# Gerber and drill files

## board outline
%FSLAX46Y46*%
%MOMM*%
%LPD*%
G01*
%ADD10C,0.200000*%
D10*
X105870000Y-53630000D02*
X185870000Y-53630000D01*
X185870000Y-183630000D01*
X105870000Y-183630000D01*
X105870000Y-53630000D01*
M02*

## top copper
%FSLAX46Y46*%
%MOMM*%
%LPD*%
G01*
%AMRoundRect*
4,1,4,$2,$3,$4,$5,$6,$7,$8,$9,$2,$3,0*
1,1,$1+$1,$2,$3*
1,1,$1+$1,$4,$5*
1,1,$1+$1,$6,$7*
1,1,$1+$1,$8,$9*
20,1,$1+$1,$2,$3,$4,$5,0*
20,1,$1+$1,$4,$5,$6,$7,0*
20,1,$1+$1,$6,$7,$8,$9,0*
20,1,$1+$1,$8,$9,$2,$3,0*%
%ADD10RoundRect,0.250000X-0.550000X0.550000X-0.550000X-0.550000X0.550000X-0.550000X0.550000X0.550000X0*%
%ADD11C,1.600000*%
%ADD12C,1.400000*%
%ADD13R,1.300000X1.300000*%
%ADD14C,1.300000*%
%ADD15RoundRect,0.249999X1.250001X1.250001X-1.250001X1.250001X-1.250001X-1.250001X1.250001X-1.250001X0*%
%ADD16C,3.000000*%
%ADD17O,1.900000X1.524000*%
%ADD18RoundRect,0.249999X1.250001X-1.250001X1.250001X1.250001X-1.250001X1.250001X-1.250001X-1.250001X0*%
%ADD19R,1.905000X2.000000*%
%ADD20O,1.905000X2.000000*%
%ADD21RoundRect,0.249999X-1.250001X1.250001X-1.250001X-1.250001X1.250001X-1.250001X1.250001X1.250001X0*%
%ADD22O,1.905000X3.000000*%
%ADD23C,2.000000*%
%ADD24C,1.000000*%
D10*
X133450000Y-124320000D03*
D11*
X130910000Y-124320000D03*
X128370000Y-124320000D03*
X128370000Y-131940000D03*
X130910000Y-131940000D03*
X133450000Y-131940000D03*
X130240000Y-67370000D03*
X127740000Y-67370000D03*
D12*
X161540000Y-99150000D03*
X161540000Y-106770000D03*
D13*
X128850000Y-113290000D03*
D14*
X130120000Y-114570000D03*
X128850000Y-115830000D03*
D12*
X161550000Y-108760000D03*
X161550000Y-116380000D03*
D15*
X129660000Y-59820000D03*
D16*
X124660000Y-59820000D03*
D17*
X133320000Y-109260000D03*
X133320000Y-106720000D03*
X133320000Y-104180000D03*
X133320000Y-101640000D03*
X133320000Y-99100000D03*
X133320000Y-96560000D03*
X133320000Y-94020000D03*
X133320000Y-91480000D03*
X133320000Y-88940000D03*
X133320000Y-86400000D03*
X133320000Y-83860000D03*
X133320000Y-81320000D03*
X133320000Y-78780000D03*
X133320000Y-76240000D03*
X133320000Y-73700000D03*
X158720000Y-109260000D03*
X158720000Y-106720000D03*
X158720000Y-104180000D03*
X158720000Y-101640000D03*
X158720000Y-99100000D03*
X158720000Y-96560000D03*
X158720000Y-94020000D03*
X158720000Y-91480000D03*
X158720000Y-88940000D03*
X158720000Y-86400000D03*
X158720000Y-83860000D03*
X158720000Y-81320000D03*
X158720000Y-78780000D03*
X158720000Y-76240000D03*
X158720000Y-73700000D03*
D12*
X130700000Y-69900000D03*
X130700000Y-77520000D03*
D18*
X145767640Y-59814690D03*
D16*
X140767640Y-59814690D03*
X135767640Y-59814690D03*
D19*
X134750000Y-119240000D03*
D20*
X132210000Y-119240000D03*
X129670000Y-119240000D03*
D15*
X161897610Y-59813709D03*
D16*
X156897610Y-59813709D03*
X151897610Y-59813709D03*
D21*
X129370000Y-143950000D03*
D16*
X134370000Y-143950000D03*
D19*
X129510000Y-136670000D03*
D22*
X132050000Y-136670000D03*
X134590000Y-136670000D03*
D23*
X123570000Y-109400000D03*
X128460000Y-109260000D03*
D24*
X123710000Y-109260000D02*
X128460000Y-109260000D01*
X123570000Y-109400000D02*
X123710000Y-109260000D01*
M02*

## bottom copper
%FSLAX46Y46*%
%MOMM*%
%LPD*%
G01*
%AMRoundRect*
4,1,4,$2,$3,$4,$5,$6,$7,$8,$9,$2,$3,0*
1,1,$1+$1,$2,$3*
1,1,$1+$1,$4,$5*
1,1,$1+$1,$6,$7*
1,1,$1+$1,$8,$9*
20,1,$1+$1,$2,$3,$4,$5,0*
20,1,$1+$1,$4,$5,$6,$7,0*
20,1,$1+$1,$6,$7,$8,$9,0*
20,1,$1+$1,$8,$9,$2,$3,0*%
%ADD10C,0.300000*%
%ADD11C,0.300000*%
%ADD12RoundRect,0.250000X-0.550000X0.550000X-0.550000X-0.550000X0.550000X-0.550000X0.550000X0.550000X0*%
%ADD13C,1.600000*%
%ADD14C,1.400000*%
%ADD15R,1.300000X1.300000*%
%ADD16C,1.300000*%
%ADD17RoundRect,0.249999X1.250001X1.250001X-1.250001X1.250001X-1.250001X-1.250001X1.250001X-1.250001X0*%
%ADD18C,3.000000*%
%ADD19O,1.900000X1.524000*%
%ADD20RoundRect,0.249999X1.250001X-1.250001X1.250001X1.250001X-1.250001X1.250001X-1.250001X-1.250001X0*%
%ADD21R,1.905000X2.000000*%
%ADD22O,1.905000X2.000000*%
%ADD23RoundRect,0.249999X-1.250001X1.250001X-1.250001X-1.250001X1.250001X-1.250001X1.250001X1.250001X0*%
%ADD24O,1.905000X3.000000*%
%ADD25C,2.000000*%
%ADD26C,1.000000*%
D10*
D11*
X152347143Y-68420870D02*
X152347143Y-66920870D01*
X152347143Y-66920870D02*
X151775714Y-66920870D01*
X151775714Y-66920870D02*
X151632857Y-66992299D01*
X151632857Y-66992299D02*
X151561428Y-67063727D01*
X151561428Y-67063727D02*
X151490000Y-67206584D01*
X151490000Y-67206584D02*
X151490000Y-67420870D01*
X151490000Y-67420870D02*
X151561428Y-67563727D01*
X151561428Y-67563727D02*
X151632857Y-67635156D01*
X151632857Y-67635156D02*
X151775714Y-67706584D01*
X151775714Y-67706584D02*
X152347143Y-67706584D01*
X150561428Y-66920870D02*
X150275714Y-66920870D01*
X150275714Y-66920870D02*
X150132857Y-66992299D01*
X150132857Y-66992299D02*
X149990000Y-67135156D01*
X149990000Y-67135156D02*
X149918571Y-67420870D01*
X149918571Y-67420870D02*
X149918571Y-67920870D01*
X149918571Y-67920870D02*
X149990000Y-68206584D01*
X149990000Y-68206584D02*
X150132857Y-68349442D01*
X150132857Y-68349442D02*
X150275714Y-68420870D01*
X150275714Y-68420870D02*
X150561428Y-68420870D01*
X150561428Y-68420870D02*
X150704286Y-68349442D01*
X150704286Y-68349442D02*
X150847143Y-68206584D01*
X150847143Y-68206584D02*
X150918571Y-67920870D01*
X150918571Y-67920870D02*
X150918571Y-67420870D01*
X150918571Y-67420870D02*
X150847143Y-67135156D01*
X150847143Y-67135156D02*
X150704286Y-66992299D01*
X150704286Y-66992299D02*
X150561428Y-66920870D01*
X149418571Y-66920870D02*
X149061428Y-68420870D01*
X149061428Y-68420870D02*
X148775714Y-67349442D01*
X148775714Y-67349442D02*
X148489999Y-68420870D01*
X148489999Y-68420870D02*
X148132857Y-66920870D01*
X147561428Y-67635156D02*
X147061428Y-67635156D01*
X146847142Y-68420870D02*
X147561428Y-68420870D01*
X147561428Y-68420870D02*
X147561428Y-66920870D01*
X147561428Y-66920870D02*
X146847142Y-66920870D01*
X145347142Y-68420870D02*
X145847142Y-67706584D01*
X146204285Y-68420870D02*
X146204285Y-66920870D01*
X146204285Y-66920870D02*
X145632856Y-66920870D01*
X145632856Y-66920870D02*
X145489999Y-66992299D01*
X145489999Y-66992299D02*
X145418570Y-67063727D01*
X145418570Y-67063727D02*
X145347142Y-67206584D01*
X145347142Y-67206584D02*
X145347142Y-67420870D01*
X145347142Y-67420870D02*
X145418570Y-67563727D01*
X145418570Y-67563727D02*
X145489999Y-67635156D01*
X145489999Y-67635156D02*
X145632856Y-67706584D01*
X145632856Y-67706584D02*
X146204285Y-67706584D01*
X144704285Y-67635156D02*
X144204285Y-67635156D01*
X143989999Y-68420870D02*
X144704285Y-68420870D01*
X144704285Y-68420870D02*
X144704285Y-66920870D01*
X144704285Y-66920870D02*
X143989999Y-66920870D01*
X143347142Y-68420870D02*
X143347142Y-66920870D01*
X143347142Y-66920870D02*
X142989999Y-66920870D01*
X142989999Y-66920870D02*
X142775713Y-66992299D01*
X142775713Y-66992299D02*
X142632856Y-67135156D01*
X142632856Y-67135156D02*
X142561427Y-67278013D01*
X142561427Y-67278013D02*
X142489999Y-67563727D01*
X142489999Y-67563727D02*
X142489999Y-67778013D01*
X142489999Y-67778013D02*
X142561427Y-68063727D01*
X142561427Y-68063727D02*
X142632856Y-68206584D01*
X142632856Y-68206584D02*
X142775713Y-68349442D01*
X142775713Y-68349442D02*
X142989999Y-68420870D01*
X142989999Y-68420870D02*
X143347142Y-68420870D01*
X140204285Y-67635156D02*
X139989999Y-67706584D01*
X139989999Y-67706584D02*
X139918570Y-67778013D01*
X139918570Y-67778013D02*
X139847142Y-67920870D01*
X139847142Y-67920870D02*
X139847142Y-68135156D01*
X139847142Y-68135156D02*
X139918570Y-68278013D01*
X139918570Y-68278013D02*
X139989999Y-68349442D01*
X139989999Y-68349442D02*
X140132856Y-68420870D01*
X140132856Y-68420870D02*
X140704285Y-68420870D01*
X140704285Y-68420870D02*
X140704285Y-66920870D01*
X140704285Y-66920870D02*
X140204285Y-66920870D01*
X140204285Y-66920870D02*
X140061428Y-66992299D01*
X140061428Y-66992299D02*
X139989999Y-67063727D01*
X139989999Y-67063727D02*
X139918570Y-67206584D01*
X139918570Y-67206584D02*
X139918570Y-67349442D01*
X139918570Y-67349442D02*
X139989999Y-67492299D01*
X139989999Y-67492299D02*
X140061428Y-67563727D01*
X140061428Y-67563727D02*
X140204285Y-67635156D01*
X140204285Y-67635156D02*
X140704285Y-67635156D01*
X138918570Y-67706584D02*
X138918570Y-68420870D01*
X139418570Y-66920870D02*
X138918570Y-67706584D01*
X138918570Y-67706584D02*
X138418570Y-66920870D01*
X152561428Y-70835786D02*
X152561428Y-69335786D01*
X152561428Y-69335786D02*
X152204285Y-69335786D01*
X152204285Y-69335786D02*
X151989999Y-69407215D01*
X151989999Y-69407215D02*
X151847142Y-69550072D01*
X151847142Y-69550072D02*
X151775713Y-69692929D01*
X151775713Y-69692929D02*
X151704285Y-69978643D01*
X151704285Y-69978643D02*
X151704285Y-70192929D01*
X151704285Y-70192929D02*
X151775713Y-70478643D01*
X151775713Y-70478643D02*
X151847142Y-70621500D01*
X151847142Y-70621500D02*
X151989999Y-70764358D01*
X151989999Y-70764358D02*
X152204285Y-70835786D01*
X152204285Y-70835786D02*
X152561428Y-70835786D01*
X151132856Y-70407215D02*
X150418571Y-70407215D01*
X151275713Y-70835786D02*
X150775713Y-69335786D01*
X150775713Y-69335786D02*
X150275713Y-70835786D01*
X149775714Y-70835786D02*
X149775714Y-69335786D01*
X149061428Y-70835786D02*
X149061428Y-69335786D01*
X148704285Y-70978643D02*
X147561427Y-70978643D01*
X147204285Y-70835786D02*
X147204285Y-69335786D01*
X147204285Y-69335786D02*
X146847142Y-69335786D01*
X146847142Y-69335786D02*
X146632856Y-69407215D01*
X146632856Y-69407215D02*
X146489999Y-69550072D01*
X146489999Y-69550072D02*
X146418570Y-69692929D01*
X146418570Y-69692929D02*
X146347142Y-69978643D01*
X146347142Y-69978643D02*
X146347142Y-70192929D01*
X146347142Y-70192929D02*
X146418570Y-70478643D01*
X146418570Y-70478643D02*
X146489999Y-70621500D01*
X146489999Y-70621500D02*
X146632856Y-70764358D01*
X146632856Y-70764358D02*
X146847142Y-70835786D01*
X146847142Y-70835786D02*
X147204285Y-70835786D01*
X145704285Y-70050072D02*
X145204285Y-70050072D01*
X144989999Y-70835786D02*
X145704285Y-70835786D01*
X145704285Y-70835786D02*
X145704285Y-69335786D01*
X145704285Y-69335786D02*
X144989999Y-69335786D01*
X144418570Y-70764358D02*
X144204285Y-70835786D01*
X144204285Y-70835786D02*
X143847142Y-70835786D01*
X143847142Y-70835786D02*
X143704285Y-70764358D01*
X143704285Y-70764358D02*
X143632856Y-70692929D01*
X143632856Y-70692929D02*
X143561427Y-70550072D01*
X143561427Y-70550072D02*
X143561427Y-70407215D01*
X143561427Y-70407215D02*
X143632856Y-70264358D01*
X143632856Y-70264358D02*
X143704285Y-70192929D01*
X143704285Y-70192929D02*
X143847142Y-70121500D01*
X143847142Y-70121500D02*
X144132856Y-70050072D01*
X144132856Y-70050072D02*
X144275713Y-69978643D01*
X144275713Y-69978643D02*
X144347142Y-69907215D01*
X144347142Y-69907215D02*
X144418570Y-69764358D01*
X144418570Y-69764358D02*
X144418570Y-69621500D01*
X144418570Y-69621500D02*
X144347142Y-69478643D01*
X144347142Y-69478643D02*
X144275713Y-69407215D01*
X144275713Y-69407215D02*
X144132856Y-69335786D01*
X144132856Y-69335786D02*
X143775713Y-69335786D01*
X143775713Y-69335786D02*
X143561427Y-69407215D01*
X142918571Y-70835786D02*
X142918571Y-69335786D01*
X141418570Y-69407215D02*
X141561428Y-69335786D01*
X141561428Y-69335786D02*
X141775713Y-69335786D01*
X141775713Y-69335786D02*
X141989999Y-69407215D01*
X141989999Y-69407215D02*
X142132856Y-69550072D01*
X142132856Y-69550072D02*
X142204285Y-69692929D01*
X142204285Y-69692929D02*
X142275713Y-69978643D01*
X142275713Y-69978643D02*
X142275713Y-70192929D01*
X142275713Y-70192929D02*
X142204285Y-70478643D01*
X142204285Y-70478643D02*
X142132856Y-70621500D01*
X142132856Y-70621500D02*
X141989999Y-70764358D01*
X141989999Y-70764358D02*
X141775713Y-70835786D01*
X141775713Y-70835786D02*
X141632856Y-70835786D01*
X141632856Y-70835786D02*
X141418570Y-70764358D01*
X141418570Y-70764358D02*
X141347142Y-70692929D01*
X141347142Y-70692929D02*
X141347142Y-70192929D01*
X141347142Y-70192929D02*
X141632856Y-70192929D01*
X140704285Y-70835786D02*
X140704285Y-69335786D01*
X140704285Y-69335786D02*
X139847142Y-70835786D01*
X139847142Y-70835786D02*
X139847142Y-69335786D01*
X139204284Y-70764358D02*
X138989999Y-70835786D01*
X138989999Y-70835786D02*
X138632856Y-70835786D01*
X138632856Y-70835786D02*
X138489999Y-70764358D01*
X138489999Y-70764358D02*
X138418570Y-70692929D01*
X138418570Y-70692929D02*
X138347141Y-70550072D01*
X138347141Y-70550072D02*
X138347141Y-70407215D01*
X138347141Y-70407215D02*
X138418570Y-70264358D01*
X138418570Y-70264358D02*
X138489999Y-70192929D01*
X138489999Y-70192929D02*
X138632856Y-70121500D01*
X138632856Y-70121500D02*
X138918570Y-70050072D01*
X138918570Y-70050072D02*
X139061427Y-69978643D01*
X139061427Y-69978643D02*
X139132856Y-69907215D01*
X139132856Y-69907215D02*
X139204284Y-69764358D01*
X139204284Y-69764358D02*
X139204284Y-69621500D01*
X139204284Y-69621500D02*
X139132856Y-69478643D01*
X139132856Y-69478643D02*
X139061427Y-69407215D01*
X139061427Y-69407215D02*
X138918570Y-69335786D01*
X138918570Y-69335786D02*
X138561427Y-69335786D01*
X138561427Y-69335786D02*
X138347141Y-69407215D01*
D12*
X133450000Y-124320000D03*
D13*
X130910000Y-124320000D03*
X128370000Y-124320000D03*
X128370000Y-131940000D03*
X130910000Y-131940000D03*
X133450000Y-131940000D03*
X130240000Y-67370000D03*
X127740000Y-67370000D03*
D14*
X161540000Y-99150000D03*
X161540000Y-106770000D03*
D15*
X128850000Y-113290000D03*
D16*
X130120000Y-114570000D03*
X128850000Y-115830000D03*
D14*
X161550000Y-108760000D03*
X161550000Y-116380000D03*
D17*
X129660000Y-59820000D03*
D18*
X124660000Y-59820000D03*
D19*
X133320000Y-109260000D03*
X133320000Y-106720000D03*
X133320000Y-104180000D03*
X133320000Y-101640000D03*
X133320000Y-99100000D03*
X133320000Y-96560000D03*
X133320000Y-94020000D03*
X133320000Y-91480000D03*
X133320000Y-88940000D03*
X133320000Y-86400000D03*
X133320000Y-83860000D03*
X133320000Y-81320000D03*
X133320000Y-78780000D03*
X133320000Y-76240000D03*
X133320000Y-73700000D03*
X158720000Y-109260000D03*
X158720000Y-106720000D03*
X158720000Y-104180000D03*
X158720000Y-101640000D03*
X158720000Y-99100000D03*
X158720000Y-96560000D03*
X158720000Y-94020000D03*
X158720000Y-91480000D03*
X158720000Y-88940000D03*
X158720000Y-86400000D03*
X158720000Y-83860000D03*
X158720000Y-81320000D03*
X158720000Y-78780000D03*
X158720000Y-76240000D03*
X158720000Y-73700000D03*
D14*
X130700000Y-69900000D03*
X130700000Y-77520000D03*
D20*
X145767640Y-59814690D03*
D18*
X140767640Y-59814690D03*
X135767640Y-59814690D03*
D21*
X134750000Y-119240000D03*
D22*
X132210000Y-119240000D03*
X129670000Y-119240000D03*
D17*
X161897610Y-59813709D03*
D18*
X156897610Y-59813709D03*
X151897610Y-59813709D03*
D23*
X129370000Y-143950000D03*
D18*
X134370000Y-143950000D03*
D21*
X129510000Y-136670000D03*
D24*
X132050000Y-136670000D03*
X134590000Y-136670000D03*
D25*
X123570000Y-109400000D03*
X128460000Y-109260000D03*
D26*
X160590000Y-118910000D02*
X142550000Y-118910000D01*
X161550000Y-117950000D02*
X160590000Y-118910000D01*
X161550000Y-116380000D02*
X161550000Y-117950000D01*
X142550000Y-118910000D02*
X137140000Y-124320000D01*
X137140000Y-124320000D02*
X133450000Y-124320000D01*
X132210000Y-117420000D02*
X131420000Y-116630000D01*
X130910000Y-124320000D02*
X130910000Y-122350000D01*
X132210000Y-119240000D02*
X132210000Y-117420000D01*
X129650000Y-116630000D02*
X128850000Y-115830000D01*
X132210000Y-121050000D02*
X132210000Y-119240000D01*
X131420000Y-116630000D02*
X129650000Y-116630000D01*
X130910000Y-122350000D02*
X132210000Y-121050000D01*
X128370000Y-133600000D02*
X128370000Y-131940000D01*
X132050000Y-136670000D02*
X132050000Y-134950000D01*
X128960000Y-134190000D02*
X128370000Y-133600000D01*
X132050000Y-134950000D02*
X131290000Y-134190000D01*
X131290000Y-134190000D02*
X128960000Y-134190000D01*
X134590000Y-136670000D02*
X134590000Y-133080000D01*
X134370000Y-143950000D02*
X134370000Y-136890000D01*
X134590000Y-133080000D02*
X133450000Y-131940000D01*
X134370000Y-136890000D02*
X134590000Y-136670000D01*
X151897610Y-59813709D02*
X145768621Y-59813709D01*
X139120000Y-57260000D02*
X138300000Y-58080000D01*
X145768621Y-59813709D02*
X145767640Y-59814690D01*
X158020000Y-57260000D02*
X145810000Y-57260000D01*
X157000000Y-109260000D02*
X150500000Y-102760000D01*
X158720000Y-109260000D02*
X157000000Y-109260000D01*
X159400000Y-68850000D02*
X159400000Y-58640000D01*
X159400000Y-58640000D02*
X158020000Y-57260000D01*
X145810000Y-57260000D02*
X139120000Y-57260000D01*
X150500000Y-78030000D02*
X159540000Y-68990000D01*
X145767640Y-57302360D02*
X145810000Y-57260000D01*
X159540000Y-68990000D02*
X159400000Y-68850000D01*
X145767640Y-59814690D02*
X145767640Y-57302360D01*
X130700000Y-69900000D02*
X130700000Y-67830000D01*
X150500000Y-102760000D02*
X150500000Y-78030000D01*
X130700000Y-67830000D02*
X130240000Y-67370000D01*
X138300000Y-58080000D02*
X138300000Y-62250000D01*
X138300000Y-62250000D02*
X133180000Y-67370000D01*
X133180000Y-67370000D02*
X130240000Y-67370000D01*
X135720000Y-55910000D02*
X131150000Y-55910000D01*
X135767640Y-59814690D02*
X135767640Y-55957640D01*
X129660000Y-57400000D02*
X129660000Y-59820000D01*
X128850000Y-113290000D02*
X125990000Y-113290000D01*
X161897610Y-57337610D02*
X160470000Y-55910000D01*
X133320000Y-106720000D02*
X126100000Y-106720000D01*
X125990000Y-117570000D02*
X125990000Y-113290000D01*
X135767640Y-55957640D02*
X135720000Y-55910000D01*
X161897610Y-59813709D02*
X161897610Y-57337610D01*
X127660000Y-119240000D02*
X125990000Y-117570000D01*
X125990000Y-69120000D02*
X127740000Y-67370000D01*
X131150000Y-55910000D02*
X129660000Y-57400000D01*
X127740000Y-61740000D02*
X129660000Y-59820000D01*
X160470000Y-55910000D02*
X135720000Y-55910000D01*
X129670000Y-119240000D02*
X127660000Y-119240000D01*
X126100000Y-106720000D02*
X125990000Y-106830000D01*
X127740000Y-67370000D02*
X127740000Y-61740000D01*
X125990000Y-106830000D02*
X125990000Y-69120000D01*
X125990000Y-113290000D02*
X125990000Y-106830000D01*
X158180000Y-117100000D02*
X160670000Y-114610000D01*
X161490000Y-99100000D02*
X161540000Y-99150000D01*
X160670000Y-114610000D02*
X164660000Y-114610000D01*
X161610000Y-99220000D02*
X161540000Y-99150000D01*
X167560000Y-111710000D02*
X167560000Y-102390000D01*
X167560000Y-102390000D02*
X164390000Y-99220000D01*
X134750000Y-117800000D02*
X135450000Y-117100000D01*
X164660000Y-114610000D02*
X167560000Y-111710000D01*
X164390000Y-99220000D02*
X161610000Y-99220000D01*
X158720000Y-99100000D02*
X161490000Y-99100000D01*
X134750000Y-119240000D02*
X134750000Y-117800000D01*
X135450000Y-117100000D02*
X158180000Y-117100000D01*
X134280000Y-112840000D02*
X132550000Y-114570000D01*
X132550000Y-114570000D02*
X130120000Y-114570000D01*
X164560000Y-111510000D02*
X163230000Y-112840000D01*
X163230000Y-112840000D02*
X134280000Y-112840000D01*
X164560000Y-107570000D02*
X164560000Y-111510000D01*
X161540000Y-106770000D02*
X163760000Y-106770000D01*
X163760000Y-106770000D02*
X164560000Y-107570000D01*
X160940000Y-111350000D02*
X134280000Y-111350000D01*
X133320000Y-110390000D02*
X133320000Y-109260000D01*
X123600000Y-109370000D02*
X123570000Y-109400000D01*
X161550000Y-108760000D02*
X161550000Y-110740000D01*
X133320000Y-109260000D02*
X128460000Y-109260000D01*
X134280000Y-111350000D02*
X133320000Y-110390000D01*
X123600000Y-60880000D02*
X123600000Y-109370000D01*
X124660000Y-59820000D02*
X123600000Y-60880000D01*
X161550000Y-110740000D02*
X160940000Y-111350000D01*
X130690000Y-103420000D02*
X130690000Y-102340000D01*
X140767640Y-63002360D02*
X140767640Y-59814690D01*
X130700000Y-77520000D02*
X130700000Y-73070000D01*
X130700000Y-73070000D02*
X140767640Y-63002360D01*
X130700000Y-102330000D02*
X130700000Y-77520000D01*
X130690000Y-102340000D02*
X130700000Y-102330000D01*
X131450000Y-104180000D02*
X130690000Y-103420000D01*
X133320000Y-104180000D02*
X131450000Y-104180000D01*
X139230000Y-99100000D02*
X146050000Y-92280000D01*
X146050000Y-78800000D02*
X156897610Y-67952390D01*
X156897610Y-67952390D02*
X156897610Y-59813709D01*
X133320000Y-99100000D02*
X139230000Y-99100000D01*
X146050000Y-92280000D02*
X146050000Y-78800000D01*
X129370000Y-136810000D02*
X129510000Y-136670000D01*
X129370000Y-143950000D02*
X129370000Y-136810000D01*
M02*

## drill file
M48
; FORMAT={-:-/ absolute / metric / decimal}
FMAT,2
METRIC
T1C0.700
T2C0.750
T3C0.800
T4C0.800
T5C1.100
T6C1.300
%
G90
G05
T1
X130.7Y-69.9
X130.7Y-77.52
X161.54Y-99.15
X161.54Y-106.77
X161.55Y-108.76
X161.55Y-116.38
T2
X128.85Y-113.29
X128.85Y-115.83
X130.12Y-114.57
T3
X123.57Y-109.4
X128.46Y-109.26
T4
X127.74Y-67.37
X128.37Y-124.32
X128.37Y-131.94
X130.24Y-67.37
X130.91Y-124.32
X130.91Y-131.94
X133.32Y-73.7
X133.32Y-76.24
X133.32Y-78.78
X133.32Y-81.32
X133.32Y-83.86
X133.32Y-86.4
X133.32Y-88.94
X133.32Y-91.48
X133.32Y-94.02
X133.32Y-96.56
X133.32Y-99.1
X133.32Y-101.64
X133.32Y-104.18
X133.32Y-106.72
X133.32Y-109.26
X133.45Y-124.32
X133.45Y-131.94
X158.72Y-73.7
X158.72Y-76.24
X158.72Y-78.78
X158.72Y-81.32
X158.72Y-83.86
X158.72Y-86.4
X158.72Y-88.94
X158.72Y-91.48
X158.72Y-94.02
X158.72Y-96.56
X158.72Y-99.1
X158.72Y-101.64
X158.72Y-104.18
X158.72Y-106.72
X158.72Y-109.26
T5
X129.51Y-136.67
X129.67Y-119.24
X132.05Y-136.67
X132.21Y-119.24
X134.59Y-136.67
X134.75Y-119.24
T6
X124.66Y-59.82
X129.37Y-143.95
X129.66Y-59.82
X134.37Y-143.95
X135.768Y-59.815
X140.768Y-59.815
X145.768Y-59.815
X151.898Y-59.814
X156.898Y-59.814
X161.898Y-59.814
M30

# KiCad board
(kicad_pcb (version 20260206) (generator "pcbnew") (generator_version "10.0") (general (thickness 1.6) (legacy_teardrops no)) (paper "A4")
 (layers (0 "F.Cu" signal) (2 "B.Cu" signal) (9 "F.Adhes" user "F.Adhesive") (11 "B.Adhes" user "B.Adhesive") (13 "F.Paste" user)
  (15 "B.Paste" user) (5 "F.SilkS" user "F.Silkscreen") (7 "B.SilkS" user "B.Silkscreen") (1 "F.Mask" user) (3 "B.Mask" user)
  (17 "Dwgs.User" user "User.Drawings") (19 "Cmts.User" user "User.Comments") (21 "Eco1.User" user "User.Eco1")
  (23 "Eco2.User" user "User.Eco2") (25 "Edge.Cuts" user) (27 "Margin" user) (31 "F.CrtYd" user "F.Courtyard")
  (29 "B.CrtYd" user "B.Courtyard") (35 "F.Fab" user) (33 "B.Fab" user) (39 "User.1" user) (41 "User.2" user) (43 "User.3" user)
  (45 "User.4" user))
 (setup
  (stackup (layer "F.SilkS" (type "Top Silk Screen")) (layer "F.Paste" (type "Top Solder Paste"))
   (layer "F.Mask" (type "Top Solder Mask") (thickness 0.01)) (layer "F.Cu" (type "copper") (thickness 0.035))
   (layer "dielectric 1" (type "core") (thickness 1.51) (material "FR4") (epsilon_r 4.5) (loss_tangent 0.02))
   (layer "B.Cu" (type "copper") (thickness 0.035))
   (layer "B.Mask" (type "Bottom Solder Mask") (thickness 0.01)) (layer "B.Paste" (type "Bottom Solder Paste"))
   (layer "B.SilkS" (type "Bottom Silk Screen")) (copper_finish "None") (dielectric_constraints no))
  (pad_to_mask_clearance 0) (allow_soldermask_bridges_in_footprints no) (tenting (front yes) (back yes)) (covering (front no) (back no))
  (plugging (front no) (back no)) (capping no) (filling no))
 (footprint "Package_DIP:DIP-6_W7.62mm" (layer "F.Cu") (at 133.45 124.32 -90)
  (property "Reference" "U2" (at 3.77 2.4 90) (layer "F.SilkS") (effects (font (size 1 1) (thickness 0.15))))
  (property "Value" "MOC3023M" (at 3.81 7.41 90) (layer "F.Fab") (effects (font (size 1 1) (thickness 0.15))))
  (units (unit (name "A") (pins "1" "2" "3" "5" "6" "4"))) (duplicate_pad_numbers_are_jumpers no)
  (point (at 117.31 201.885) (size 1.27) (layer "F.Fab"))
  (pad "1" thru_hole roundrect (at 0 0 270) (size 1.6 1.6) (drill 0.8) (layers "*.Cu" "*.Mask") (remove_unused_layers no)
   (roundrect_rratio 0.15625) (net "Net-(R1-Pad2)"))
  (pad "2" thru_hole circle (at 0 2.54 270) (size 1.6 1.6) (drill 0.8) (layers "*.Cu" "*.Mask") (remove_unused_layers no) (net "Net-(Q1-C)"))
  (pad "3" thru_hole circle (at 0 5.08 270) (size 1.6 1.6) (drill 0.8) (layers "*.Cu" "*.Mask") (remove_unused_layers no)
   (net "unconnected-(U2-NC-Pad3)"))
  (pad "4" thru_hole circle (at 7.62 5.08 270) (size 1.6 1.6) (drill 0.8) (layers "*.Cu" "*.Mask") (remove_unused_layers no)
   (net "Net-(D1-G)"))
  (pad "5" thru_hole circle (at 7.62 2.54 270) (size 1.6 1.6) (drill 0.8) (layers "*.Cu" "*.Mask") (remove_unused_layers no)
   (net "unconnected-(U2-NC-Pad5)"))
  (pad "6" thru_hole circle (at 7.62 0 270) (size 1.6 1.6) (drill 0.8) (layers "*.Cu" "*.Mask") (remove_unused_layers no)
   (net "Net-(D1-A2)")))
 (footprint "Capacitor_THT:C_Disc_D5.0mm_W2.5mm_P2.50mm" (layer "F.Cu") (at 130.24 67.37 180)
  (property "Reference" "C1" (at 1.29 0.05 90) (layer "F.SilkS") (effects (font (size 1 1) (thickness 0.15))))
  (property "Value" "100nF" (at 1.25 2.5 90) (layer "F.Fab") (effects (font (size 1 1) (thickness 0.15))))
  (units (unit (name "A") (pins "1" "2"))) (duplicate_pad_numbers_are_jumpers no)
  (pad "1" thru_hole circle (at 0 0 90) (size 1.6 1.6) (drill 0.8) (layers "*.Cu" "*.Mask") (remove_unused_layers no) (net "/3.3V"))
  (pad "2" thru_hole circle (at 2.5 0 90) (size 1.6 1.6) (drill 0.8) (layers "*.Cu" "*.Mask") (remove_unused_layers no) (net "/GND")))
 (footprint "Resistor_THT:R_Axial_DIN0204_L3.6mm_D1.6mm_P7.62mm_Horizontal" (layer "F.Cu") (at 161.54 99.15 -90)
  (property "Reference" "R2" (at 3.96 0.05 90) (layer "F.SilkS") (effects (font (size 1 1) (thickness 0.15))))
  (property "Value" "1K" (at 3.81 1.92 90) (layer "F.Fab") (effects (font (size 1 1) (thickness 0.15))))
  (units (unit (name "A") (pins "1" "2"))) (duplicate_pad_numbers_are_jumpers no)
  (pad "1" thru_hole circle (at 0 0 270) (size 1.4 1.4) (drill 0.7) (layers "*.Cu" "*.Mask") (remove_unused_layers no) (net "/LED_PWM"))
  (pad "2" thru_hole circle (at 7.62 0 270) (size 1.4 1.4) (drill 0.7) (layers "*.Cu" "*.Mask") (remove_unused_layers no) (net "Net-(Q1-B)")))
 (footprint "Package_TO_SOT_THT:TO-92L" (layer "F.Cu") (at 128.85 113.29 -90)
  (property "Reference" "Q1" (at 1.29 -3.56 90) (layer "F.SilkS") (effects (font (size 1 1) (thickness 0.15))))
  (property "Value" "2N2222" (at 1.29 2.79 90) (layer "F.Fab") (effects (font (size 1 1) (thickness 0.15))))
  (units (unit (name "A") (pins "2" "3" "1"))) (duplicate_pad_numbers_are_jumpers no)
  (pad "1" thru_hole rect (at 0 0 270) (size 1.3 1.3) (drill 0.75) (layers "*.Cu" "*.Mask") (remove_unused_layers no) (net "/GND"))
  (pad "2" thru_hole circle (at 1.28 -1.27 270) (size 1.3 1.3) (drill 0.75) (layers "*.Cu" "*.Mask") (remove_unused_layers no)
   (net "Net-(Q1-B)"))
  (pad "3" thru_hole circle (at 2.54 0 270) (size 1.3 1.3) (drill 0.75) (layers "*.Cu" "*.Mask") (remove_unused_layers no)
   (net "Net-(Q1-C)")))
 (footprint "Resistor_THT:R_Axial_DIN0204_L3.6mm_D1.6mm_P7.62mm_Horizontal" (layer "F.Cu") (at 161.55 108.76 -90)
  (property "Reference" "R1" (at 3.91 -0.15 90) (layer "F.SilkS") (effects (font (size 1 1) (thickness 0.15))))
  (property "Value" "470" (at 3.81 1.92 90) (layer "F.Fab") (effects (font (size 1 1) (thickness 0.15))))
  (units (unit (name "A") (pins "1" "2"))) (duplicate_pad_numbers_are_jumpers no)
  (pad "1" thru_hole circle (at 0 0 270) (size 1.4 1.4) (drill 0.7) (layers "*.Cu" "*.Mask") (remove_unused_layers no) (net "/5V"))
  (pad "2" thru_hole circle (at 7.62 0 270) (size 1.4 1.4) (drill 0.7) (layers "*.Cu" "*.Mask") (remove_unused_layers no)
   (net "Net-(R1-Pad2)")))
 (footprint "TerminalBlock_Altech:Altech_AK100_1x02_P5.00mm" (layer "F.Cu") (at 129.66 59.82 180)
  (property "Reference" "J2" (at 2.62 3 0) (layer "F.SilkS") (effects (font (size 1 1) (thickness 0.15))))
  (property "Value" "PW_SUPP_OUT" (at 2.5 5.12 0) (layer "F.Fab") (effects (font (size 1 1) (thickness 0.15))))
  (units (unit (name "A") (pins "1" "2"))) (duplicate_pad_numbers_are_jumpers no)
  (pad "1" thru_hole roundrect (at 0 0 180) (size 3 3) (drill 1.3) (layers "*.Cu" "*.Mask") (remove_unused_layers no)
   (roundrect_rratio 0.083333) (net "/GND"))
  (pad "2" thru_hole circle (at 5 0 180) (size 3 3) (drill 1.3) (layers "*.Cu" "*.Mask") (remove_unused_layers no) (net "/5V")))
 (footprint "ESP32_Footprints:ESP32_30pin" (layer "F.Cu") (at 145.24754 92.240187)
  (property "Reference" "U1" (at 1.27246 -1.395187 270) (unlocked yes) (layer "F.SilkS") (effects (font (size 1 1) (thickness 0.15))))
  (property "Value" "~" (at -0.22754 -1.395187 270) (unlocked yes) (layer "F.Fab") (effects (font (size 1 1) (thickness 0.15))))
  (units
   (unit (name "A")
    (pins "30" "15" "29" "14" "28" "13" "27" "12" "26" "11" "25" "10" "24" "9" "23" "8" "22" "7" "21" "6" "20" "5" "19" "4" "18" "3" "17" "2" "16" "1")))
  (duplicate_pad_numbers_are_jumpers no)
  (pad "1" thru_hole oval (at -11.92754 17.019813 270) (size 1.524 1.9) (drill 0.8) (layers "*.Cu" "*.Mask") (remove_unused_layers no)
   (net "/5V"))
  (pad "2" thru_hole oval (at -11.92754 14.479813 270) (size 1.524 1.9) (drill 0.8) (layers "*.Cu" "*.Mask") (remove_unused_layers no)
   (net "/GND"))
  (pad "3" thru_hole oval (at -11.92754 11.939813 270) (size 1.524 1.9) (drill 0.8) (layers "*.Cu" "*.Mask") (remove_unused_layers no)
   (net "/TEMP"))
  (pad "4" thru_hole oval (at -11.92754 9.399813 270) (size 1.524 1.9) (drill 0.8) (layers "*.Cu" "*.Mask") (remove_unused_layers no)
   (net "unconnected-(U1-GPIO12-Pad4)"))
  (pad "5" thru_hole oval (at -11.92754 6.859813 270) (size 1.524 1.9) (drill 0.8) (layers "*.Cu" "*.Mask") (remove_unused_layers no)
   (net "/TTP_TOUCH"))
  (pad "6" thru_hole oval (at -11.92754 4.319813 270) (size 1.524 1.9) (drill 0.8) (layers "*.Cu" "*.Mask") (remove_unused_layers no)
   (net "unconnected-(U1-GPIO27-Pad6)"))
  (pad "7" thru_hole oval (at -11.92754 1.779813 270) (size 1.524 1.9) (drill 0.8) (layers "*.Cu" "*.Mask") (remove_unused_layers no)
   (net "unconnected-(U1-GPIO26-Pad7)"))
  (pad "8" thru_hole oval (at -11.92754 -0.760187 270) (size 1.524 1.9) (drill 0.8) (layers "*.Cu" "*.Mask") (remove_unused_layers no)
   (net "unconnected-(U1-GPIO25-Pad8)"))
  (pad "9" thru_hole oval (at -11.92754 -3.300187 270) (size 1.524 1.9) (drill 0.8) (layers "*.Cu" "*.Mask") (remove_unused_layers no)
   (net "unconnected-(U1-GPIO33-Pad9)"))
  (pad "10" thru_hole oval (at -11.92754 -5.840187 270) (size 1.524 1.9) (drill 0.8) (layers "*.Cu" "*.Mask") (remove_unused_layers no)
   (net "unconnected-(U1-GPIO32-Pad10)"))
  (pad "11" thru_hole oval (at -11.92754 -8.380187 270) (size 1.524 1.9) (drill 0.8) (layers "*.Cu" "*.Mask") (remove_unused_layers no)
   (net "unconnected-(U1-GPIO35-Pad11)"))
  (pad "12" thru_hole oval (at -11.92754 -10.920187 270) (size 1.524 1.9) (drill 0.8) (layers "*.Cu" "*.Mask") (remove_unused_layers no)
   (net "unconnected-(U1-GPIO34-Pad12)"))
  (pad "13" thru_hole oval (at -11.92754 -13.460187 270) (size 1.524 1.9) (drill 0.8) (layers "*.Cu" "*.Mask") (remove_unused_layers no)
   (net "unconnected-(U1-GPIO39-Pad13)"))
  (pad "14" thru_hole oval (at -11.92754 -16.000187 270) (size 1.524 1.9) (drill 0.8) (layers "*.Cu" "*.Mask") (remove_unused_layers no)
   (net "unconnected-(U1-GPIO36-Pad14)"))
  (pad "15" thru_hole oval (at -11.92754 -18.540187 270) (size 1.524 1.9) (drill 0.8) (layers "*.Cu" "*.Mask") (remove_unused_layers no)
   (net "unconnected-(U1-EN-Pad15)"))
  (pad "16" thru_hole oval (at 13.47246 17.019813 270) (size 1.524 1.9) (drill 0.8) (layers "*.Cu" "*.Mask") (remove_unused_layers no)
   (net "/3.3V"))
  (pad "17" thru_hole oval (at 13.47246 14.479813 270) (size 1.524 1.9) (drill 0.8) (layers "*.Cu" "*.Mask") (remove_unused_layers no)
   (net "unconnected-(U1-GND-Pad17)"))
  (pad "18" thru_hole oval (at 13.47246 11.939813 270) (size 1.524 1.9) (drill 0.8) (layers "*.Cu" "*.Mask") (remove_unused_layers no)
   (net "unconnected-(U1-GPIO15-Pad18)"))
  (pad "19" thru_hole oval (at 13.47246 9.399813 270) (size 1.524 1.9) (drill 0.8) (layers "*.Cu" "*.Mask") (remove_unused_layers no)
   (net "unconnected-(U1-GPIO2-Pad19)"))
  (pad "20" thru_hole oval (at 13.47246 6.859813 270) (size 1.524 1.9) (drill 0.8) (layers "*.Cu" "*.Mask" "Dwgs.User")
   (remove_unused_layers no) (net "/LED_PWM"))
  (pad "21" thru_hole oval (at 13.47246 4.319813 270) (size 1.524 1.9) (drill 0.8) (layers "*.Cu" "*.Mask") (remove_unused_layers no)
   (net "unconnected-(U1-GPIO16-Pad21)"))
  (pad "22" thru_hole oval (at 13.47246 1.779813 270) (size 1.524 1.9) (drill 0.8) (layers "*.Cu" "*.Mask") (remove_unused_layers no)
   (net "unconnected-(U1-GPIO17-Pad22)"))
  (pad "23" thru_hole oval (at 13.47246 -0.760187 270) (size 1.524 1.9) (drill 0.8) (layers "*.Cu" "*.Mask") (remove_unused_layers no)
   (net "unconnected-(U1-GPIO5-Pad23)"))
  (pad "24" thru_hole oval (at 13.47246 -3.300187 270) (size 1.524 1.9) (drill 0.8) (layers "*.Cu" "*.Mask") (remove_unused_layers no)
   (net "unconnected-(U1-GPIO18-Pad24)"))
  (pad "25" thru_hole oval (at 13.47246 -5.840187 270) (size 1.524 1.9) (drill 0.8) (layers "*.Cu" "*.Mask") (remove_unused_layers no)
   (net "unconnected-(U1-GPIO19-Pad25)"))
  (pad "26" thru_hole oval (at 13.47246 -8.380187 270) (size 1.524 1.9) (drill 0.8) (layers "*.Cu" "*.Mask") (remove_unused_layers no)
   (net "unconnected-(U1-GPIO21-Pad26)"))
  (pad "27" thru_hole oval (at 13.47246 -10.920187 270) (size 1.524 1.9) (drill 0.8) (layers "*.Cu" "*.Mask") (remove_unused_layers no)
   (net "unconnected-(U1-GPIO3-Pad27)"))
  (pad "28" thru_hole oval (at 13.47246 -13.460187 270) (size 1.524 1.9) (drill 0.8) (layers "*.Cu" "*.Mask") (remove_unused_layers no)
   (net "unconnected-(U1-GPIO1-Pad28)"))
  (pad "29" thru_hole oval (at 13.47246 -16.000187 270) (size 1.524 1.9) (drill 0.8) (layers "*.Cu" "*.Mask") (remove_unused_layers no)
   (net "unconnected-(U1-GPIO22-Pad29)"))
  (pad "30" thru_hole oval (at 13.47246 -18.540187 270) (size 1.524 1.9) (drill 0.8) (layers "*.Cu" "*.Mask") (remove_unused_layers no)
   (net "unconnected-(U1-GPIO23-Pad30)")))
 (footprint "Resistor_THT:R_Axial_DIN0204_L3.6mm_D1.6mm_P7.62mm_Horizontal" (layer "F.Cu") (at 130.7 69.9 -90)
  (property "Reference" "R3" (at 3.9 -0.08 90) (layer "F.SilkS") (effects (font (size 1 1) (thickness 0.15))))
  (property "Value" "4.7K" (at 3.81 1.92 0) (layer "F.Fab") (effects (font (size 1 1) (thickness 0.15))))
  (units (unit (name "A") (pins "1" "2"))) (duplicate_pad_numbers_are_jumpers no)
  (pad "1" thru_hole circle (at 0 0 180) (size 1.4 1.4) (drill 0.7) (layers "*.Cu" "*.Mask") (remove_unused_layers no) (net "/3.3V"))
  (pad "2" thru_hole circle (at 7.62 0 180) (size 1.4 1.4) (drill 0.7) (layers "*.Cu" "*.Mask") (remove_unused_layers no) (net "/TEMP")))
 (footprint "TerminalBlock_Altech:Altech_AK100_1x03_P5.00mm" (layer "F.Cu") (at 145.76764 59.81469 180)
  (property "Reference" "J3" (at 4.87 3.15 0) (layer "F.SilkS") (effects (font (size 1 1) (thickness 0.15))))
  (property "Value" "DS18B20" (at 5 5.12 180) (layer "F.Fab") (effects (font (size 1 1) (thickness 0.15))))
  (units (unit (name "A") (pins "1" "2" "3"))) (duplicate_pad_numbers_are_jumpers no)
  (pad "1" thru_hole roundrect (at 0 0 90) (size 3 3) (drill 1.3) (layers "*.Cu" "*.Mask") (remove_unused_layers no)
   (roundrect_rratio 0.083333) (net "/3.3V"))
  (pad "2" thru_hole circle (at 5 0 90) (size 3 3) (drill 1.3) (layers "*.Cu" "*.Mask") (remove_unused_layers no) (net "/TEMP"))
  (pad "3" thru_hole circle (at 10 0 90) (size 3 3) (drill 1.3) (layers "*.Cu" "*.Mask") (remove_unused_layers no) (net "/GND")))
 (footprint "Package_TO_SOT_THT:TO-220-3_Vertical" (layer "F.Cu") (at 134.75 119.24 180)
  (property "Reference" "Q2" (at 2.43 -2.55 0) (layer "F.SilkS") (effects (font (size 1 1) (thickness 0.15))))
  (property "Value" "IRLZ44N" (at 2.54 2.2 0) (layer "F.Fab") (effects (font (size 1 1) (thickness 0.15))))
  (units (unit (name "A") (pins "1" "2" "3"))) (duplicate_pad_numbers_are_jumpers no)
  (pad "1" thru_hole rect (at 0 0 180) (size 1.905 2) (drill 1.1) (layers "*.Cu" "*.Mask") (remove_unused_layers no) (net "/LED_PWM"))
  (pad "2" thru_hole oval (at 2.54 0 180) (size 1.905 2) (drill 1.1) (layers "*.Cu" "*.Mask") (remove_unused_layers no) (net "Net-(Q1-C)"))
  (pad "3" thru_hole oval (at 5.08 0 180) (size 1.905 2) (drill 1.1) (layers "*.Cu" "*.Mask") (remove_unused_layers no) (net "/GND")))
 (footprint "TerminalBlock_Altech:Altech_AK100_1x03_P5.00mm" (layer "F.Cu") (at 161.89761 59.813709 180)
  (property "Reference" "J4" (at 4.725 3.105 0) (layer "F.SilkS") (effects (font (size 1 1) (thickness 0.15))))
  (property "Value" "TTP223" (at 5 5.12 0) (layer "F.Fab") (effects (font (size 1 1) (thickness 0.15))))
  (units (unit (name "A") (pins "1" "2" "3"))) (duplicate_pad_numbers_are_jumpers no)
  (pad "1" thru_hole roundrect (at 0 0 180) (size 3 3) (drill 1.3) (layers "*.Cu" "*.Mask") (remove_unused_layers no)
   (roundrect_rratio 0.083333) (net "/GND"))
  (pad "2" thru_hole circle (at 5 0 180) (size 3 3) (drill 1.3) (layers "*.Cu" "*.Mask") (remove_unused_layers no) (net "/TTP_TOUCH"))
  (pad "3" thru_hole circle (at 10 0 180) (size 3 3) (drill 1.3) (layers "*.Cu" "*.Mask") (remove_unused_layers no) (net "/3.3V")))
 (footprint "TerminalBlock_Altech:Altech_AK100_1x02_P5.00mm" (layer "F.Cu") (at 129.37 143.95)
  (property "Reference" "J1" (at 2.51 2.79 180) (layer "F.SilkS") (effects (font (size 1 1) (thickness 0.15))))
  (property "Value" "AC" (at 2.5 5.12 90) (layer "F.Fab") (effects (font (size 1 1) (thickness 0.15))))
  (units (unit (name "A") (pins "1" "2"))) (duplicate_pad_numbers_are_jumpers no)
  (pad "1" thru_hole roundrect (at 0 0 270) (size 3 3) (drill 1.3) (layers "*.Cu" "*.Mask") (remove_unused_layers no)
   (roundrect_rratio 0.083333) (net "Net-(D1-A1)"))
  (pad "2" thru_hole circle (at 5 0 270) (size 3 3) (drill 1.3) (layers "*.Cu" "*.Mask") (remove_unused_layers no) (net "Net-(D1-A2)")))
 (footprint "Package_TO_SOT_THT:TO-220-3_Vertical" (layer "F.Cu") (at 129.51 136.67)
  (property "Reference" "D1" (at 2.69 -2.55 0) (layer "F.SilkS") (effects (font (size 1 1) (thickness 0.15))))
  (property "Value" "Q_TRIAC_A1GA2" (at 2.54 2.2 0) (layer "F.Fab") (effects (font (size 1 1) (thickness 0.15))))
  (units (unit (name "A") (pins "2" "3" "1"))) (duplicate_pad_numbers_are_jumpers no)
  (pad "1" thru_hole rect (at 0 0) (size 1.905 2) (drill 1.1) (layers "*.Cu" "*.Mask") (remove_unused_layers no) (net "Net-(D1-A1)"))
  (pad "2" thru_hole oval (at 2.54 0) (size 1.905 3) (drill 1.1) (layers "*.Cu" "*.Mask") (remove_unused_layers no) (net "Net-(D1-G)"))
  (pad "3" thru_hole oval (at 5.08 0) (size 1.905 3) (drill 1.1) (layers "*.Cu" "*.Mask") (remove_unused_layers no) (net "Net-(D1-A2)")))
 (gr_rect (start 105.87 53.63) (end 185.87 183.63) (stroke (width 0.2) (type solid)) (fill no) (layer "Edge.Cuts"))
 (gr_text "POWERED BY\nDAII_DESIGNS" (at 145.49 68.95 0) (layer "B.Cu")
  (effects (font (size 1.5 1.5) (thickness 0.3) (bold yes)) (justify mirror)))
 (segment (start 160.59 118.91) (end 142.55 118.91) (width 1) (layer "B.Cu") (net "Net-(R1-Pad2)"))
 (segment (start 161.55 117.95) (end 160.59 118.91) (width 1) (layer "B.Cu") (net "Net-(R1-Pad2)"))
 (segment (start 161.55 116.38) (end 161.55 117.95) (width 1) (layer "B.Cu") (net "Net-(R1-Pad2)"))
 (segment (start 142.55 118.91) (end 137.14 124.32) (width 1) (layer "B.Cu") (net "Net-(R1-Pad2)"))
 (segment (start 137.14 124.32) (end 133.45 124.32) (width 1) (layer "B.Cu") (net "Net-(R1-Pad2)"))
 (segment (start 132.21 117.42) (end 131.42 116.63) (width 1) (layer "B.Cu") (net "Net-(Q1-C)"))
 (segment (start 130.91 124.32) (end 130.91 122.35) (width 1) (layer "B.Cu") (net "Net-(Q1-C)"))
 (segment (start 132.21 119.24) (end 132.21 117.42) (width 1) (layer "B.Cu") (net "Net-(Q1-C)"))
 (segment (start 129.65 116.63) (end 128.85 115.83) (width 1) (layer "B.Cu") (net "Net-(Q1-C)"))
 (segment (start 132.21 121.05) (end 132.21 119.24) (width 1) (layer "B.Cu") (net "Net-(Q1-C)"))
 (segment (start 131.42 116.63) (end 129.65 116.63) (width 1) (layer "B.Cu") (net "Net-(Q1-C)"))
 (segment (start 130.91 122.35) (end 132.21 121.05) (width 1) (layer "B.Cu") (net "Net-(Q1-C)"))
 (segment (start 128.37 133.6) (end 128.37 131.94) (width 1) (layer "B.Cu") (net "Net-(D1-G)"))
 (segment (start 132.05 136.67) (end 132.05 134.95) (width 1) (layer "B.Cu") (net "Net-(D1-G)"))
 (segment (start 128.96 134.19) (end 128.37 133.6) (width 1) (layer "B.Cu") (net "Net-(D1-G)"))
 (segment (start 132.05 134.95) (end 131.29 134.19) (width 1) (layer "B.Cu") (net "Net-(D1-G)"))
 (segment (start 131.29 134.19) (end 128.96 134.19) (width 1) (layer "B.Cu") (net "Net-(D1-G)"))
 (segment (start 134.59 136.67) (end 134.59 133.08) (width 1) (layer "B.Cu") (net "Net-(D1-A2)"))
 (segment (start 134.37 143.95) (end 134.37 136.89) (width 1) (layer "B.Cu") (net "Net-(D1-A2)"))
 (segment (start 134.59 133.08) (end 133.45 131.94) (width 1) (layer "B.Cu") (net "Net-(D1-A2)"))
 (segment (start 134.37 136.89) (end 134.59 136.67) (width 1) (layer "B.Cu") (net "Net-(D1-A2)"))
 (segment (start 151.89761 59.813709) (end 145.768621 59.813709) (width 1) (layer "B.Cu") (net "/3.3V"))
 (segment (start 139.12 57.26) (end 138.3 58.08) (width 1) (layer "B.Cu") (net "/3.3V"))
 (segment (start 145.768621 59.813709) (end 145.76764 59.81469) (width 1) (layer "B.Cu") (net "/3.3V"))
 (segment (start 158.02 57.26) (end 145.81 57.26) (width 1) (layer "B.Cu") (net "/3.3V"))
 (segment (start 157 109.26) (end 150.5 102.76) (width 1) (layer "B.Cu") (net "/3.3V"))
 (segment (start 158.72 109.26) (end 157 109.26) (width 1) (layer "B.Cu") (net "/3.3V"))
 (segment (start 159.4 68.85) (end 159.4 58.64) (width 1) (layer "B.Cu") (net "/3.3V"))
 (segment (start 159.4 58.64) (end 158.02 57.26) (width 1) (layer "B.Cu") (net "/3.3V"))
 (segment (start 145.81 57.26) (end 139.12 57.26) (width 1) (layer "B.Cu") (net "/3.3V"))
 (segment (start 150.5 78.03) (end 159.54 68.99) (width 1) (layer "B.Cu") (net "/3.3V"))
 (segment (start 145.76764 57.30236) (end 145.81 57.26) (width 1) (layer "B.Cu") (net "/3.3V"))
 (segment (start 159.54 68.99) (end 159.4 68.85) (width 1) (layer "B.Cu") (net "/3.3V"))
 (segment (start 145.76764 59.81469) (end 145.76764 57.30236) (width 1) (layer "B.Cu") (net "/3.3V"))
 (segment (start 130.7 69.9) (end 130.7 67.83) (width 1) (layer "B.Cu") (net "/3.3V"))
 (segment (start 150.5 102.76) (end 150.5 78.03) (width 1) (layer "B.Cu") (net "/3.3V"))
 (segment (start 130.7 67.83) (end 130.24 67.37) (width 1) (layer "B.Cu") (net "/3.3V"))
 (segment (start 138.3 58.08) (end 138.3 62.25) (width 1) (layer "B.Cu") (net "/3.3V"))
 (segment (start 138.3 62.25) (end 133.18 67.37) (width 1) (layer "B.Cu") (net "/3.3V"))
 (segment (start 133.18 67.37) (end 130.24 67.37) (width 1) (layer "B.Cu") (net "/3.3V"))
 (segment (start 135.72 55.91) (end 131.15 55.91) (width 1) (layer "B.Cu") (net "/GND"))
 (segment (start 135.76764 59.81469) (end 135.76764 55.95764) (width 1) (layer "B.Cu") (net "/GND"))
 (segment (start 129.66 57.4) (end 129.66 59.82) (width 1) (layer "B.Cu") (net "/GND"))
 (segment (start 128.85 113.29) (end 125.99 113.29) (width 1) (layer "B.Cu") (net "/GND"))
 (segment (start 161.89761 57.33761) (end 160.47 55.91) (width 1) (layer "B.Cu") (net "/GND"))
 (segment (start 133.32 106.72) (end 126.1 106.72) (width 1) (layer "B.Cu") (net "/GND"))
 (segment (start 125.99 117.57) (end 125.99 113.29) (width 1) (layer "B.Cu") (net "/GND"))
 (segment (start 135.76764 55.95764) (end 135.72 55.91) (width 1) (layer "B.Cu") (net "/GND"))
 (segment (start 161.89761 59.813709) (end 161.89761 57.33761) (width 1) (layer "B.Cu") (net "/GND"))
 (segment (start 127.66 119.24) (end 125.99 117.57) (width 1) (layer "B.Cu") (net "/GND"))
 (segment (start 125.99 69.12) (end 127.74 67.37) (width 1) (layer "B.Cu") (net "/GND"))
 (segment (start 131.15 55.91) (end 129.66 57.4) (width 1) (layer "B.Cu") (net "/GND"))
 (segment (start 127.74 61.74) (end 129.66 59.82) (width 1) (layer "B.Cu") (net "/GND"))
 (segment (start 160.47 55.91) (end 135.72 55.91) (width 1) (layer "B.Cu") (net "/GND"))
 (segment (start 129.67 119.24) (end 127.66 119.24) (width 1) (layer "B.Cu") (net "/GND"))
 (segment (start 126.1 106.72) (end 125.99 106.83) (width 1) (layer "B.Cu") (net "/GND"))
 (segment (start 127.74 67.37) (end 127.74 61.74) (width 1) (layer "B.Cu") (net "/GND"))
 (segment (start 125.99 106.83) (end 125.99 69.12) (width 1) (layer "B.Cu") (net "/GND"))
 (segment (start 125.99 113.29) (end 125.99 106.83) (width 1) (layer "B.Cu") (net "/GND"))
 (segment (start 158.18 117.1) (end 160.67 114.61) (width 1) (layer "B.Cu") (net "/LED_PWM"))
 (segment (start 161.49 99.1) (end 161.54 99.15) (width 1) (layer "B.Cu") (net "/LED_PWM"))
 (segment (start 160.67 114.61) (end 164.66 114.61) (width 1) (layer "B.Cu") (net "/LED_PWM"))
 (segment (start 161.61 99.22) (end 161.54 99.15) (width 1) (layer "B.Cu") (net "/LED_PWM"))
 (segment (start 167.56 111.71) (end 167.56 102.39) (width 1) (layer "B.Cu") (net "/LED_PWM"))
 (segment (start 167.56 102.39) (end 164.39 99.22) (width 1) (layer "B.Cu") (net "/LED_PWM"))
 (segment (start 134.75 117.8) (end 135.45 117.1) (width 1) (layer "B.Cu") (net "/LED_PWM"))
 (segment (start 164.66 114.61) (end 167.56 111.71) (width 1) (layer "B.Cu") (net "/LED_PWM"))
 (segment (start 164.39 99.22) (end 161.61 99.22) (width 1) (layer "B.Cu") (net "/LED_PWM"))
 (segment (start 158.72 99.1) (end 161.49 99.1) (width 1) (layer "B.Cu") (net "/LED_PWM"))
 (segment (start 134.75 119.24) (end 134.75 117.8) (width 1) (layer "B.Cu") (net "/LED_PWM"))
 (segment (start 135.45 117.1) (end 158.18 117.1) (width 1) (layer "B.Cu") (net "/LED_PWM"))
 (segment (start 134.28 112.84) (end 132.55 114.57) (width 1) (layer "B.Cu") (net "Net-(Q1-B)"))
 (segment (start 132.55 114.57) (end 130.12 114.57) (width 1) (layer "B.Cu") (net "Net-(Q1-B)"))
 (segment (start 164.56 111.51) (end 163.23 112.84) (width 1) (layer "B.Cu") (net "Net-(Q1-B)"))
 (segment (start 163.23 112.84) (end 134.28 112.84) (width 1) (layer "B.Cu") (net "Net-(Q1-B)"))
 (segment (start 164.56 107.57) (end 164.56 111.51) (width 1) (layer "B.Cu") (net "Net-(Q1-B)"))
 (segment (start 161.54 106.77) (end 163.76 106.77) (width 1) (layer "B.Cu") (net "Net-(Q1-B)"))
 (segment (start 163.76 106.77) (end 164.56 107.57) (width 1) (layer "B.Cu") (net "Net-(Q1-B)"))
 (segment (start 123.71 109.26) (end 128.46 109.26) (width 1) (layer "F.Cu") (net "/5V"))
 (segment (start 123.57 109.4) (end 123.71 109.26) (width 1) (layer "F.Cu") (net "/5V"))
 (via (at 123.57 109.4) (size 2) (drill 0.8) (layers "F.Cu" "B.Cu") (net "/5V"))
 (via (at 128.46 109.26) (size 2) (drill 0.8) (layers "F.Cu" "B.Cu") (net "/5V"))
 (segment (start 160.94 111.35) (end 134.28 111.35) (width 1) (layer "B.Cu") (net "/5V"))
 (segment (start 133.32 110.39) (end 133.32 109.26) (width 1) (layer "B.Cu") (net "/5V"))
 (segment (start 123.6 109.37) (end 123.57 109.4) (width 1) (layer "B.Cu") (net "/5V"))
 (segment (start 161.55 108.76) (end 161.55 110.74) (width 1) (layer "B.Cu") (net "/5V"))
 (segment (start 133.32 109.26) (end 128.46 109.26) (width 1) (layer "B.Cu") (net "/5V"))
 (segment (start 134.28 111.35) (end 133.32 110.39) (width 1) (layer "B.Cu") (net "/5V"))
 (segment (start 123.6 60.88) (end 123.6 109.37) (width 1) (layer "B.Cu") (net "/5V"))
 (segment (start 124.66 59.82) (end 123.6 60.88) (width 1) (layer "B.Cu") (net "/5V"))
 (segment (start 161.55 110.74) (end 160.94 111.35) (width 1) (layer "B.Cu") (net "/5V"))
 (segment (start 130.69 103.42) (end 130.69 102.34) (width 1) (layer "B.Cu") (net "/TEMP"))
 (segment (start 140.76764 63.00236) (end 140.76764 59.81469) (width 1) (layer "B.Cu") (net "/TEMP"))
 (segment (start 130.7 77.52) (end 130.7 73.07) (width 1) (layer "B.Cu") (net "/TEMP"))
 (segment (start 130.7 73.07) (end 140.76764 63.00236) (width 1) (layer "B.Cu") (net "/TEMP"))
 (segment (start 130.7 102.33) (end 130.7 77.52) (width 1) (layer "B.Cu") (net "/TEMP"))
 (segment (start 130.69 102.34) (end 130.7 102.33) (width 1) (layer "B.Cu") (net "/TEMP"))
 (segment (start 131.45 104.18) (end 130.69 103.42) (width 1) (layer "B.Cu") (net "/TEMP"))
 (segment (start 133.32 104.18) (end 131.45 104.18) (width 1) (layer "B.Cu") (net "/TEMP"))
 (segment (start 139.23 99.1) (end 146.05 92.28) (width 1) (layer "B.Cu") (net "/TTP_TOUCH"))
 (segment (start 146.05 78.8) (end 156.89761 67.95239) (width 1) (layer "B.Cu") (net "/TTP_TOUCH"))
 (segment (start 156.89761 67.95239) (end 156.89761 59.813709) (width 1) (layer "B.Cu") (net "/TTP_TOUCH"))
 (segment (start 133.32 99.1) (end 139.23 99.1) (width 1) (layer "B.Cu") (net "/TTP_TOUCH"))
 (segment (start 146.05 92.28) (end 146.05 78.8) (width 1) (layer "B.Cu") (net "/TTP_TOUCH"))
 (segment (start 129.37 136.81) (end 129.51 136.67) (width 1) (layer "B.Cu") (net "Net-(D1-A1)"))
 (segment (start 129.37 143.95) (end 129.37 136.81) (width 1) (layer "B.Cu") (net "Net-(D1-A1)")))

